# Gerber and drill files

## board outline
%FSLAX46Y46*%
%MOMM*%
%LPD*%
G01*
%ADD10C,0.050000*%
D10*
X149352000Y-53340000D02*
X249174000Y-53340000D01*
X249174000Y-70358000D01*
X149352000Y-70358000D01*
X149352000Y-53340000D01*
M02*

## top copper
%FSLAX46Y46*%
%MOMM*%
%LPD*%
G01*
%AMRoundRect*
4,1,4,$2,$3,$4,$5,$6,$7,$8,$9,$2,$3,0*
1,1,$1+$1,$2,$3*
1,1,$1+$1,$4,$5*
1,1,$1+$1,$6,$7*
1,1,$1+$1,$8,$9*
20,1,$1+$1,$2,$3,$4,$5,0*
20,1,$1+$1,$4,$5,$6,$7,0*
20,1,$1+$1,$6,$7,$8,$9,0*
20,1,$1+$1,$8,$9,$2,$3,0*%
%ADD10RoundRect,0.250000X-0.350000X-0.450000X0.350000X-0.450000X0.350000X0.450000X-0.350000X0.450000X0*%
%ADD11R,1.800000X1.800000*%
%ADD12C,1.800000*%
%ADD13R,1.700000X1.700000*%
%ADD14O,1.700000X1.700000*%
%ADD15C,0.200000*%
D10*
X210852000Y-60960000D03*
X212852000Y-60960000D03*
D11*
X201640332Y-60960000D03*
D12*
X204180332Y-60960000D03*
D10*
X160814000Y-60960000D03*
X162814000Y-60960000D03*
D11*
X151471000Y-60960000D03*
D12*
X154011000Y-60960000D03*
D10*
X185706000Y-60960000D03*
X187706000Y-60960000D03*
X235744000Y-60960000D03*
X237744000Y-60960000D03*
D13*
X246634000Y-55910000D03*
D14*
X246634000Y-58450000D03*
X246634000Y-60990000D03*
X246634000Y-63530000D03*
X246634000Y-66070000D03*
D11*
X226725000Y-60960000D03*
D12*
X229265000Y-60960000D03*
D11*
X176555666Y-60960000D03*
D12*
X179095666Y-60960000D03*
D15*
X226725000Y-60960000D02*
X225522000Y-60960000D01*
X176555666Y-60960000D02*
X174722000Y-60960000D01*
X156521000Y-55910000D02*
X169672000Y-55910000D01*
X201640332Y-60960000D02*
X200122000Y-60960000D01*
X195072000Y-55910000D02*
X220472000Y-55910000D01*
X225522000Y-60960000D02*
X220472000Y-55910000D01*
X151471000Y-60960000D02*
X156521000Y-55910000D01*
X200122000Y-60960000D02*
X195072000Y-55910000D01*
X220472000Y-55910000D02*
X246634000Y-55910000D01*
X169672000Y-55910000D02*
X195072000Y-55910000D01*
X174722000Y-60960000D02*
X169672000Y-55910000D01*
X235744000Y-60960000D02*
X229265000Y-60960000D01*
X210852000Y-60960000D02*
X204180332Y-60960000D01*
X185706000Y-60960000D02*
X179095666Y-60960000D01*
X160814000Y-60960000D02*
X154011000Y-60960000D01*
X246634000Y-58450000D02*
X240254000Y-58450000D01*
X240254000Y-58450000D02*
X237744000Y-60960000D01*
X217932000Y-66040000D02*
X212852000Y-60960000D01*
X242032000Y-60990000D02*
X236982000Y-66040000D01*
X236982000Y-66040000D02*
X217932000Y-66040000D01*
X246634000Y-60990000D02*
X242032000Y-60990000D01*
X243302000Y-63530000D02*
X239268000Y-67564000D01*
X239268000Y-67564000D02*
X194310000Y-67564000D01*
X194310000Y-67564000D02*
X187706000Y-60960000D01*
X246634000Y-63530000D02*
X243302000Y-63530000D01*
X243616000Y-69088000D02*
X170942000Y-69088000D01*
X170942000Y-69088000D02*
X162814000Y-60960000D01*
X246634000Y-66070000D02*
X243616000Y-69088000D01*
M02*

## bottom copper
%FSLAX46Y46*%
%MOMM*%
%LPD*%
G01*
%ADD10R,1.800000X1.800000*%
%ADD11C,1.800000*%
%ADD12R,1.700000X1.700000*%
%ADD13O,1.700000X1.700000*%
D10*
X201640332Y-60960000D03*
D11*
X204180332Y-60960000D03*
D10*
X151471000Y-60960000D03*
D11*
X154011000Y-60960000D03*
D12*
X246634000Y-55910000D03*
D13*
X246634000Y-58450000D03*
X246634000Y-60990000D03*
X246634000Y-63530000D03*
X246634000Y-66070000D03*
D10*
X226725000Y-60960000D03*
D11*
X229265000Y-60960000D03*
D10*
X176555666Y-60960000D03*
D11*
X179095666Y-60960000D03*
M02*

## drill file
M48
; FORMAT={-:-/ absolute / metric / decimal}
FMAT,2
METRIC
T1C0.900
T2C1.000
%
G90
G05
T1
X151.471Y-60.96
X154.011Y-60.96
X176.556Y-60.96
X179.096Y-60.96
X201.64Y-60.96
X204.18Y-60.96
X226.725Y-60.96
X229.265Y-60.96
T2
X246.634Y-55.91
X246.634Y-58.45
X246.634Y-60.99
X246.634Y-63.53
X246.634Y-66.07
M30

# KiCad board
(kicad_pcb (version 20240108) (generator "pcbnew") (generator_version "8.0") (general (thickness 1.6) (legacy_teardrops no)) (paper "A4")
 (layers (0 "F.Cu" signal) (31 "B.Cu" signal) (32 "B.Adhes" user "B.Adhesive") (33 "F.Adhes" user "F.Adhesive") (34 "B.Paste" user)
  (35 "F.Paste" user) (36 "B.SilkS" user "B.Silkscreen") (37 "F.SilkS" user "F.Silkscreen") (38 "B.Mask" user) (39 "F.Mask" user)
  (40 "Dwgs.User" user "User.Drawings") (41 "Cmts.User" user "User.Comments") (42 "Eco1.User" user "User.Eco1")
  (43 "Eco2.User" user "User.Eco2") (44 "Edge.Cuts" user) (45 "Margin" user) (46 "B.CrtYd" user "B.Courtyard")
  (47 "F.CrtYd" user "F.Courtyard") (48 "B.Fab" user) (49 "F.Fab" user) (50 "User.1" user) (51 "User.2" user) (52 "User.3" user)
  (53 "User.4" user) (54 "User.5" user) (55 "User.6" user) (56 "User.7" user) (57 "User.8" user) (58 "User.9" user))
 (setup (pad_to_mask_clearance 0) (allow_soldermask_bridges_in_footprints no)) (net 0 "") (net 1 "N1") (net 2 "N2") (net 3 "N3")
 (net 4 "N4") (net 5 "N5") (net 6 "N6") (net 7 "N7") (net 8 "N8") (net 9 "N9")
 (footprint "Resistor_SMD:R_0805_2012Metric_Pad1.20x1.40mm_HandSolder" (layer "F.Cu") (at 211.852 60.96)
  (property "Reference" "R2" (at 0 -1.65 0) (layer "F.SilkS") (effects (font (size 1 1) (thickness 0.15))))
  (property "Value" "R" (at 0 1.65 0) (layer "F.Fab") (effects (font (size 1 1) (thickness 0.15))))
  (pad "1" smd roundrect (at -1 0) (size 1.2 1.4) (layers "F.Cu" "F.Paste" "F.Mask") (roundrect_rratio 0.208333) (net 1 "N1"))
  (pad "2" smd roundrect (at 1 0) (size 1.2 1.4) (layers "F.Cu" "F.Paste" "F.Mask") (roundrect_rratio 0.208333) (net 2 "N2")))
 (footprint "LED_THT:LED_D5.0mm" (layer "F.Cu") (at 201.640332 60.96)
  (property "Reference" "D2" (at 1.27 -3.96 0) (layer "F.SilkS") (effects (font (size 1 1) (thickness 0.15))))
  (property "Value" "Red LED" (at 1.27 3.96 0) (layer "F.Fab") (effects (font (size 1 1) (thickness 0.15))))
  (pad "1" thru_hole rect (at 0 0) (size 1.8 1.8) (drill 0.9) (layers "*.Cu" "*.Mask") (remove_unused_layers no) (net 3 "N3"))
  (pad "2" thru_hole circle (at 2.54 0) (size 1.8 1.8) (drill 0.9) (layers "*.Cu" "*.Mask") (remove_unused_layers no) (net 1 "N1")))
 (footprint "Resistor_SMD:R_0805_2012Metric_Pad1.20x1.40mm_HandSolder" (layer "F.Cu") (at 161.814 60.96)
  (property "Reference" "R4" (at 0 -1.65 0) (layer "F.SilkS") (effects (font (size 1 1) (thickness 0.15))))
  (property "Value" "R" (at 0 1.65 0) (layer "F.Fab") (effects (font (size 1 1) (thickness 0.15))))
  (pad "1" smd roundrect (at -1 0) (size 1.2 1.4) (layers "F.Cu" "F.Paste" "F.Mask") (roundrect_rratio 0.208333) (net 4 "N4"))
  (pad "2" smd roundrect (at 1 0) (size 1.2 1.4) (layers "F.Cu" "F.Paste" "F.Mask") (roundrect_rratio 0.208333) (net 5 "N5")))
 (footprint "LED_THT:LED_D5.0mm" (layer "F.Cu") (at 151.471 60.96)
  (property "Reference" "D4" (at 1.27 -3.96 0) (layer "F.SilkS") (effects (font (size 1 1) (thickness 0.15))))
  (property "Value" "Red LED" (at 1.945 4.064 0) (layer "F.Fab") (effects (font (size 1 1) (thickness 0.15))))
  (pad "1" thru_hole rect (at 0 0) (size 1.8 1.8) (drill 0.9) (layers "*.Cu" "*.Mask") (remove_unused_layers no) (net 3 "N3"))
  (pad "2" thru_hole circle (at 2.54 0) (size 1.8 1.8) (drill 0.9) (layers "*.Cu" "*.Mask") (remove_unused_layers no) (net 4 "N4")))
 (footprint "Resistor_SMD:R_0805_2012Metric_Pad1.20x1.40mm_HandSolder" (layer "F.Cu") (at 186.706 60.96)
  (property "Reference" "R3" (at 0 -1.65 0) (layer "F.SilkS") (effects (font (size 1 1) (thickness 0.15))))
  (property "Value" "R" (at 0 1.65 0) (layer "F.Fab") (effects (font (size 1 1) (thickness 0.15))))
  (pad "1" smd roundrect (at -1 0) (size 1.2 1.4) (layers "F.Cu" "F.Paste" "F.Mask") (roundrect_rratio 0.208333) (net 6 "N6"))
  (pad "2" smd roundrect (at 1 0) (size 1.2 1.4) (layers "F.Cu" "F.Paste" "F.Mask") (roundrect_rratio 0.208333) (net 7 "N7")))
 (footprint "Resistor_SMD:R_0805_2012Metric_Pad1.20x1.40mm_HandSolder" (layer "F.Cu") (at 236.744 60.96)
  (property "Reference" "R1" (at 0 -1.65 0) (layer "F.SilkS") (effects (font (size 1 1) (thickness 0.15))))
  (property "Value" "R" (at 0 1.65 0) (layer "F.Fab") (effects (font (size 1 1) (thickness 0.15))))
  (pad "1" smd roundrect (at -1 0) (size 1.2 1.4) (layers "F.Cu" "F.Paste" "F.Mask") (roundrect_rratio 0.208333) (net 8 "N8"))
  (pad "2" smd roundrect (at 1 0) (size 1.2 1.4) (layers "F.Cu" "F.Paste" "F.Mask") (roundrect_rratio 0.208333) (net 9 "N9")))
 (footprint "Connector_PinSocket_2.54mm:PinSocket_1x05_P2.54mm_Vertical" (layer "F.Cu") (at 246.634 55.91)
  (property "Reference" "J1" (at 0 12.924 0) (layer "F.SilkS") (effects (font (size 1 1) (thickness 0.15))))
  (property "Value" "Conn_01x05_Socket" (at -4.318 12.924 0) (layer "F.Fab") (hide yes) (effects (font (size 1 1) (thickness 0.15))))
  (pad "1" thru_hole rect (at 0 0) (size 1.7 1.7) (drill 1) (layers "*.Cu" "*.Mask") (remove_unused_layers no) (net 3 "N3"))
  (pad "2" thru_hole oval (at 0 2.54) (size 1.7 1.7) (drill 1) (layers "*.Cu" "*.Mask") (remove_unused_layers no) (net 9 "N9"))
  (pad "3" thru_hole oval (at 0 5.08) (size 1.7 1.7) (drill 1) (layers "*.Cu" "*.Mask") (remove_unused_layers no) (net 2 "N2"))
  (pad "4" thru_hole oval (at 0 7.62) (size 1.7 1.7) (drill 1) (layers "*.Cu" "*.Mask") (remove_unused_layers no) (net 7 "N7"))
  (pad "5" thru_hole oval (at 0 10.16) (size 1.7 1.7) (drill 1) (layers "*.Cu" "*.Mask") (remove_unused_layers no) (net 5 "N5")))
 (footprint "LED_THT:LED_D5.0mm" (layer "F.Cu") (at 226.725 60.96)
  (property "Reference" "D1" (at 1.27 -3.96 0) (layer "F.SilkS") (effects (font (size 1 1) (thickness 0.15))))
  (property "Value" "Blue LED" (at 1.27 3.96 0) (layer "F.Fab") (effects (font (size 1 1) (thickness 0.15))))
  (pad "1" thru_hole rect (at 0 0) (size 1.8 1.8) (drill 0.9) (layers "*.Cu" "*.Mask") (remove_unused_layers no) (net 3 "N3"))
  (pad "2" thru_hole circle (at 2.54 0) (size 1.8 1.8) (drill 0.9) (layers "*.Cu" "*.Mask") (remove_unused_layers no) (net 8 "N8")))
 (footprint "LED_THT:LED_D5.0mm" (layer "F.Cu") (at 176.555666 60.96)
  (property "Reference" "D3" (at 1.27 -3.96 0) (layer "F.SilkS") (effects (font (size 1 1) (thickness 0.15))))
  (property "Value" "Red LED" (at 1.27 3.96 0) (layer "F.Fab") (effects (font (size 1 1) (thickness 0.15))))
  (pad "1" thru_hole rect (at 0 0) (size 1.8 1.8) (drill 0.9) (layers "*.Cu" "*.Mask") (remove_unused_layers no) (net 3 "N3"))
  (pad "2" thru_hole circle (at 2.54 0) (size 1.8 1.8) (drill 0.9) (layers "*.Cu" "*.Mask") (remove_unused_layers no) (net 6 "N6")))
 (gr_rect (start 149.352 53.34) (end 249.174 70.358) (stroke (width 0.05) (type default)) (fill none) (layer "Edge.Cuts"))
 (segment (start 226.725 60.96) (end 225.522 60.96) (width 0.2) (layer "F.Cu") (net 3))
 (segment (start 176.555666 60.96) (end 174.722 60.96) (width 0.2) (layer "F.Cu") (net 3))
 (segment (start 156.521 55.91) (end 169.672 55.91) (width 0.2) (layer "F.Cu") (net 3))
 (segment (start 201.640332 60.96) (end 200.122 60.96) (width 0.2) (layer "F.Cu") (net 3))
 (segment (start 195.072 55.91) (end 220.472 55.91) (width 0.2) (layer "F.Cu") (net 3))
 (segment (start 225.522 60.96) (end 220.472 55.91) (width 0.2) (layer "F.Cu") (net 3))
 (segment (start 151.471 60.96) (end 156.521 55.91) (width 0.2) (layer "F.Cu") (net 3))
 (segment (start 200.122 60.96) (end 195.072 55.91) (width 0.2) (layer "F.Cu") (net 3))
 (segment (start 220.472 55.91) (end 246.634 55.91) (width 0.2) (layer "F.Cu") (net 3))
 (segment (start 169.672 55.91) (end 195.072 55.91) (width 0.2) (layer "F.Cu") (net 3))
 (segment (start 174.722 60.96) (end 169.672 55.91) (width 0.2) (layer "F.Cu") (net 3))
 (segment (start 235.744 60.96) (end 229.265 60.96) (width 0.2) (layer "F.Cu") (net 8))
 (segment (start 210.852 60.96) (end 204.180332 60.96) (width 0.2) (layer "F.Cu") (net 1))
 (segment (start 185.706 60.96) (end 179.095666 60.96) (width 0.2) (layer "F.Cu") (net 6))
 (segment (start 160.814 60.96) (end 154.011 60.96) (width 0.2) (layer "F.Cu") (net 4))
 (segment (start 246.634 58.45) (end 240.254 58.45) (width 0.2) (layer "F.Cu") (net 9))
 (segment (start 240.254 58.45) (end 237.744 60.96) (width 0.2) (layer "F.Cu") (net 9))
 (segment (start 217.932 66.04) (end 212.852 60.96) (width 0.2) (layer "F.Cu") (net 2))
 (segment (start 242.032 60.99) (end 236.982 66.04) (width 0.2) (layer "F.Cu") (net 2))
 (segment (start 236.982 66.04) (end 217.932 66.04) (width 0.2) (layer "F.Cu") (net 2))
 (segment (start 246.634 60.99) (end 242.032 60.99) (width 0.2) (layer "F.Cu") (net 2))
 (segment (start 243.302 63.53) (end 239.268 67.564) (width 0.2) (layer "F.Cu") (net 7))
 (segment (start 239.268 67.564) (end 194.31 67.564) (width 0.2) (layer "F.Cu") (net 7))
 (segment (start 194.31 67.564) (end 187.706 60.96) (width 0.2) (layer "F.Cu") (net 7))
 (segment (start 246.634 63.53) (end 243.302 63.53) (width 0.2) (layer "F.Cu") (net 7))
 (segment (start 243.616 69.088) (end 170.942 69.088) (width 0.2) (layer "F.Cu") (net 5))
 (segment (start 170.942 69.088) (end 162.814 60.96) (width 0.2) (layer "F.Cu") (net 5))
 (segment (start 246.634 66.07) (end 243.616 69.088) (width 0.2) (layer "F.Cu") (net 5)))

